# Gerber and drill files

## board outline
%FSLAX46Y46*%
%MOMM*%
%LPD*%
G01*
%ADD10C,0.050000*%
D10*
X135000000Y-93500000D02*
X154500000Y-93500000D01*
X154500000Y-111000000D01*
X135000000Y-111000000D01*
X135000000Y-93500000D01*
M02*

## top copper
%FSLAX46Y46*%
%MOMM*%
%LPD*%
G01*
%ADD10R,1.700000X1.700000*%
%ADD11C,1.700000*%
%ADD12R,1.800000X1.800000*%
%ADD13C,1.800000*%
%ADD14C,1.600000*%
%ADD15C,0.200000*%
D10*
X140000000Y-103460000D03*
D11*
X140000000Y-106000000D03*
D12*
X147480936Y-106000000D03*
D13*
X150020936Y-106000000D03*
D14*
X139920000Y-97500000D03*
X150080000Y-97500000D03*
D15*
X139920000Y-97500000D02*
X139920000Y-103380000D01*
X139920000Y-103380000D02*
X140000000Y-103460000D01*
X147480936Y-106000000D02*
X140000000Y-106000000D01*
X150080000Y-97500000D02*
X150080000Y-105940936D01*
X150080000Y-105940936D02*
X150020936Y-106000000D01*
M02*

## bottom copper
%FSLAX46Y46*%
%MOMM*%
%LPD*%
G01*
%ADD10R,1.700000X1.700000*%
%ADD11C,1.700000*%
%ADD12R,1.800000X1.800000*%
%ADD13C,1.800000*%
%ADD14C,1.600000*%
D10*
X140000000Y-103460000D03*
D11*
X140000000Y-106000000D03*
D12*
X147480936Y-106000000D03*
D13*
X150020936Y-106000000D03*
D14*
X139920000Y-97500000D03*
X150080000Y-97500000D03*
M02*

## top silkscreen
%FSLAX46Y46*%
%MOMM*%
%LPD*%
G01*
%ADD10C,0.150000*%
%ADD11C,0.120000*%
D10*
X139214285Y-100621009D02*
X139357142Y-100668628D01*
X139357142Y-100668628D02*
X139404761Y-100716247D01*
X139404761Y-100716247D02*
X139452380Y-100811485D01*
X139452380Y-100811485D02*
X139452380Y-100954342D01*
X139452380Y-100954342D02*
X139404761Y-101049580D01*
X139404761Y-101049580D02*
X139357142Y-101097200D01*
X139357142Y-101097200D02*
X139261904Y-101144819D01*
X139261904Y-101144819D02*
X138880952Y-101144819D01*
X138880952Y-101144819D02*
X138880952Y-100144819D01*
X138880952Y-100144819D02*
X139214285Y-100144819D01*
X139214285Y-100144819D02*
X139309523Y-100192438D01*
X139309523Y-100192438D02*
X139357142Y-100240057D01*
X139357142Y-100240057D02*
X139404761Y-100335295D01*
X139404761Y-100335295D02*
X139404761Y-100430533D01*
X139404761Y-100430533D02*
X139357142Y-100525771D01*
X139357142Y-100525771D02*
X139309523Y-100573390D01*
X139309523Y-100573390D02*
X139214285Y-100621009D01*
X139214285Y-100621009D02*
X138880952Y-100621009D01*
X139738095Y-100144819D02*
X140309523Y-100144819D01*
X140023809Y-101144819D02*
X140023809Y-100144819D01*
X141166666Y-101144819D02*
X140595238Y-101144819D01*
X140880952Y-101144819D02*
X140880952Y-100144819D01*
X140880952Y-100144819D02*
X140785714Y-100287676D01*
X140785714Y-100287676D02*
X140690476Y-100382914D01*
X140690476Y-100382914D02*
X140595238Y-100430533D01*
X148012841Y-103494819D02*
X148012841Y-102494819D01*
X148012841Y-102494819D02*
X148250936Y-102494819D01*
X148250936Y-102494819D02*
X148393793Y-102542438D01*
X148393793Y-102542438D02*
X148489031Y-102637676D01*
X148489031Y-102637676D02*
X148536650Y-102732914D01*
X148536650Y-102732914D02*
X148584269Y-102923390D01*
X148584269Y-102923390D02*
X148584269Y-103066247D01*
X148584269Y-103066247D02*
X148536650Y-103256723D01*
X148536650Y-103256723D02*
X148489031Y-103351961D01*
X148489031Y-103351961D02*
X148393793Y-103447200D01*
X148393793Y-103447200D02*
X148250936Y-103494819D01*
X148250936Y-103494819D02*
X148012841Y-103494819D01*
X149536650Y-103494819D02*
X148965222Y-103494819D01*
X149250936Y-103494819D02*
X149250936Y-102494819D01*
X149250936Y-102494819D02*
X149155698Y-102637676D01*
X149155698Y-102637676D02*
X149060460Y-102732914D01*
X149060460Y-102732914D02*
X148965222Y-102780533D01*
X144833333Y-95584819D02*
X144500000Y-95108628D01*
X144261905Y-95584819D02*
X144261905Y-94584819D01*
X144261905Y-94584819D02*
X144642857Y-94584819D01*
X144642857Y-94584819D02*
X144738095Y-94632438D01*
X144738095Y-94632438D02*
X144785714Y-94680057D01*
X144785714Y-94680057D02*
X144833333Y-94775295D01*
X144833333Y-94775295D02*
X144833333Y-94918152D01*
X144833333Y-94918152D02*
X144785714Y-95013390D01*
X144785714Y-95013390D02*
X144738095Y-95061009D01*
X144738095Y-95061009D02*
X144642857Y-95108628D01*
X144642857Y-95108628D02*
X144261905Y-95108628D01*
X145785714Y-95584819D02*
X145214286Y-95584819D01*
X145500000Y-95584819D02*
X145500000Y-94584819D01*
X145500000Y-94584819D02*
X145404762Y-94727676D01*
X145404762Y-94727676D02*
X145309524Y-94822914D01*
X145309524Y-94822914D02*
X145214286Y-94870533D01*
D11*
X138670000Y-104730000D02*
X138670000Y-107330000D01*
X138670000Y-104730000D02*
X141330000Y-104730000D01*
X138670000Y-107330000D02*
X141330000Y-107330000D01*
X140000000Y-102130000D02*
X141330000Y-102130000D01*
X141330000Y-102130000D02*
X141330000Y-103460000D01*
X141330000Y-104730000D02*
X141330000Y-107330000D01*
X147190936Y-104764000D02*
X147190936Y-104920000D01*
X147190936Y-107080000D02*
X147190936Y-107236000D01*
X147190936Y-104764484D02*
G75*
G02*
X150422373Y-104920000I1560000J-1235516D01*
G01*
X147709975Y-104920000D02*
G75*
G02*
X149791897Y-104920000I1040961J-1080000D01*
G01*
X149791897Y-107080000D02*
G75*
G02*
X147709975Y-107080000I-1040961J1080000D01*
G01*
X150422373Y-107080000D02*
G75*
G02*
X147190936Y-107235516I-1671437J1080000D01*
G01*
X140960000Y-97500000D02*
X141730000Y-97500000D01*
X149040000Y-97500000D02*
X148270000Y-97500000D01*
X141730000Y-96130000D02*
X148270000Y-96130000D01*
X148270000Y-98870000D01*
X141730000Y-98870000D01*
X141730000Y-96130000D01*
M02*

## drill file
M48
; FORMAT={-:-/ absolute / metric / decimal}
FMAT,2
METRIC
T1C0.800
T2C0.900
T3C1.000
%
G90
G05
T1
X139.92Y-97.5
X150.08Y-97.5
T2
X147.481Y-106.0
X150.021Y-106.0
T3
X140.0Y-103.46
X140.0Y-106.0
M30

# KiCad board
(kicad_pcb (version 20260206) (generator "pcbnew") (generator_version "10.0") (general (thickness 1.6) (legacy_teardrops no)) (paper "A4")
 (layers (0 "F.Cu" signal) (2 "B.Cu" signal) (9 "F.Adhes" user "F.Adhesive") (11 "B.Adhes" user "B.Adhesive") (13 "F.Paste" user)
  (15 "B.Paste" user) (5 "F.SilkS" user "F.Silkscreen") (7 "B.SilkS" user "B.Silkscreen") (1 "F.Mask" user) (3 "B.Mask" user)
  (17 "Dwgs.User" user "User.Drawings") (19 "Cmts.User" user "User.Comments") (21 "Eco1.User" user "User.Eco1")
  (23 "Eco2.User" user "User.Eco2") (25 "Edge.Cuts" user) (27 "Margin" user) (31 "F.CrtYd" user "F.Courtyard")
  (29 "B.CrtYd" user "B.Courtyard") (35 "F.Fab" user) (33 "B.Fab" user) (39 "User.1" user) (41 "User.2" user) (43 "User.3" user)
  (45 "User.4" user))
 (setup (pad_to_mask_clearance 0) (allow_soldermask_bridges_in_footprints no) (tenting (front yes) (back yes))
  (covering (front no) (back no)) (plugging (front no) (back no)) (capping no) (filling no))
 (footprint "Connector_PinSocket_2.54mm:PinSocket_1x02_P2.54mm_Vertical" (layer "F.Cu") (at 140 103.46)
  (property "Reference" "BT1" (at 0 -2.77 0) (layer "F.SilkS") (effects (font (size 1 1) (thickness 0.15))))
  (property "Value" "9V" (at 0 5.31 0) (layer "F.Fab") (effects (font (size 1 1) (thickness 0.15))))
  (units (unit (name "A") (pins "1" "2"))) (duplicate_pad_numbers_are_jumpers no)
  (fp_line (start -1.33 1.27) (end -1.33 3.87) (stroke (width 0.12) (type solid)) (layer "F.SilkS"))
  (fp_line (start -1.33 1.27) (end 1.33 1.27) (stroke (width 0.12) (type solid)) (layer "F.SilkS"))
  (fp_line (start -1.33 3.87) (end 1.33 3.87) (stroke (width 0.12) (type solid)) (layer "F.SilkS"))
  (fp_line (start 0 -1.33) (end 1.33 -1.33) (stroke (width 0.12) (type solid)) (layer "F.SilkS"))
  (fp_line (start 1.33 -1.33) (end 1.33 0) (stroke (width 0.12) (type solid)) (layer "F.SilkS"))
  (fp_line (start 1.33 1.27) (end 1.33 3.87) (stroke (width 0.12) (type solid)) (layer "F.SilkS"))
  (pad "1" thru_hole rect (at 0 0) (size 1.7 1.7) (drill 1) (layers "*.Cu" "*.Mask") (remove_unused_layers no) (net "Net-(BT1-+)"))
  (pad "2" thru_hole circle (at 0 2.54) (size 1.7 1.7) (drill 1) (layers "*.Cu" "*.Mask") (remove_unused_layers no) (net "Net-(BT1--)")))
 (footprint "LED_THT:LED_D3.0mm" (layer "F.Cu") (at 147.480936 106)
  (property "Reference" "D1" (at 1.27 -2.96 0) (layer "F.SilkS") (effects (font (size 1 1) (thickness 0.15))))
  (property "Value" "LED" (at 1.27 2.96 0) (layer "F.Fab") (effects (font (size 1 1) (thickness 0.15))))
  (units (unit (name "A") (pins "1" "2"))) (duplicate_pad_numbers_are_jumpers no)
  (fp_line (start -0.29 -1.236) (end -0.29 -1.08) (stroke (width 0.12) (type solid)) (layer "F.SilkS"))
  (fp_line (start -0.29 1.08) (end -0.29 1.236) (stroke (width 0.12) (type solid)) (layer "F.SilkS"))
  (fp_arc (start -0.29 -1.235516) (mid 1.36566 -1.987699) (end 2.941437 -1.08) (stroke (width 0.12) (type solid)) (layer "F.SilkS"))
  (fp_arc (start 0.229039 -1.08) (mid 1.27 -1.5) (end 2.310961 -1.08) (stroke (width 0.12) (type solid)) (layer "F.SilkS"))
  (fp_arc (start 2.310961 1.08) (mid 1.27 1.5) (end 0.229039 1.08) (stroke (width 0.12) (type solid)) (layer "F.SilkS"))
  (fp_arc (start 2.941437 1.08) (mid 1.36566 1.987699) (end -0.29 1.235516) (stroke (width 0.12) (type solid)) (layer "F.SilkS"))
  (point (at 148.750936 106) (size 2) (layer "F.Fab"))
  (pad "1" thru_hole rect (at 0 0) (size 1.8 1.8) (drill 0.9) (layers "*.Cu" "*.Mask") (remove_unused_layers no) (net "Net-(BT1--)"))
  (pad "2" thru_hole circle (at 2.54 0) (size 1.8 1.8) (drill 0.9) (layers "*.Cu" "*.Mask") (remove_unused_layers no) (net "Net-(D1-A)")))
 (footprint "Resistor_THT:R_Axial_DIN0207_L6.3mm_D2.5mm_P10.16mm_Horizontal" (layer "F.Cu") (at 139.92 97.5)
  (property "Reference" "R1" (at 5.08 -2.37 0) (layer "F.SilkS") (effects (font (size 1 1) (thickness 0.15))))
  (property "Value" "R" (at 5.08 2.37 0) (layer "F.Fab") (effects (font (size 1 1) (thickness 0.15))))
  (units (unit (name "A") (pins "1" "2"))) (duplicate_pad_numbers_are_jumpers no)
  (fp_line (start 1.04 0) (end 1.81 0) (stroke (width 0.12) (type solid)) (layer "F.SilkS"))
  (fp_line (start 9.12 0) (end 8.35 0) (stroke (width 0.12) (type solid)) (layer "F.SilkS"))
  (fp_rect (start 1.81 -1.37) (end 8.35 1.37) (stroke (width 0.12) (type solid)) (fill no) (layer "F.SilkS"))
  (pad "1" thru_hole circle (at 0 0) (size 1.6 1.6) (drill 0.8) (layers "*.Cu" "*.Mask") (remove_unused_layers no) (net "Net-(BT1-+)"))
  (pad "2" thru_hole circle (at 10.16 0) (size 1.6 1.6) (drill 0.8) (layers "*.Cu" "*.Mask") (remove_unused_layers no) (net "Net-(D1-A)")))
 (gr_rect (start 135 93.5) (end 154.5 111) (stroke (width 0.05) (type default)) (fill no) (layer "Edge.Cuts"))
 (segment (start 139.92 97.5) (end 139.92 103.38) (width 0.2) (layer "F.Cu") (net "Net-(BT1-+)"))
 (segment (start 139.92 103.38) (end 140 103.46) (width 0.2) (layer "F.Cu") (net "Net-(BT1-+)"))
 (segment (start 147.480936 106) (end 140 106) (width 0.2) (layer "F.Cu") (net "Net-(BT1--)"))
 (segment (start 150.08 97.5) (end 150.08 105.940936) (width 0.2) (layer "F.Cu") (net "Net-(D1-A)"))
 (segment (start 150.08 105.940936) (end 150.020936 106) (width 0.2) (layer "F.Cu") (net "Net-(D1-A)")))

